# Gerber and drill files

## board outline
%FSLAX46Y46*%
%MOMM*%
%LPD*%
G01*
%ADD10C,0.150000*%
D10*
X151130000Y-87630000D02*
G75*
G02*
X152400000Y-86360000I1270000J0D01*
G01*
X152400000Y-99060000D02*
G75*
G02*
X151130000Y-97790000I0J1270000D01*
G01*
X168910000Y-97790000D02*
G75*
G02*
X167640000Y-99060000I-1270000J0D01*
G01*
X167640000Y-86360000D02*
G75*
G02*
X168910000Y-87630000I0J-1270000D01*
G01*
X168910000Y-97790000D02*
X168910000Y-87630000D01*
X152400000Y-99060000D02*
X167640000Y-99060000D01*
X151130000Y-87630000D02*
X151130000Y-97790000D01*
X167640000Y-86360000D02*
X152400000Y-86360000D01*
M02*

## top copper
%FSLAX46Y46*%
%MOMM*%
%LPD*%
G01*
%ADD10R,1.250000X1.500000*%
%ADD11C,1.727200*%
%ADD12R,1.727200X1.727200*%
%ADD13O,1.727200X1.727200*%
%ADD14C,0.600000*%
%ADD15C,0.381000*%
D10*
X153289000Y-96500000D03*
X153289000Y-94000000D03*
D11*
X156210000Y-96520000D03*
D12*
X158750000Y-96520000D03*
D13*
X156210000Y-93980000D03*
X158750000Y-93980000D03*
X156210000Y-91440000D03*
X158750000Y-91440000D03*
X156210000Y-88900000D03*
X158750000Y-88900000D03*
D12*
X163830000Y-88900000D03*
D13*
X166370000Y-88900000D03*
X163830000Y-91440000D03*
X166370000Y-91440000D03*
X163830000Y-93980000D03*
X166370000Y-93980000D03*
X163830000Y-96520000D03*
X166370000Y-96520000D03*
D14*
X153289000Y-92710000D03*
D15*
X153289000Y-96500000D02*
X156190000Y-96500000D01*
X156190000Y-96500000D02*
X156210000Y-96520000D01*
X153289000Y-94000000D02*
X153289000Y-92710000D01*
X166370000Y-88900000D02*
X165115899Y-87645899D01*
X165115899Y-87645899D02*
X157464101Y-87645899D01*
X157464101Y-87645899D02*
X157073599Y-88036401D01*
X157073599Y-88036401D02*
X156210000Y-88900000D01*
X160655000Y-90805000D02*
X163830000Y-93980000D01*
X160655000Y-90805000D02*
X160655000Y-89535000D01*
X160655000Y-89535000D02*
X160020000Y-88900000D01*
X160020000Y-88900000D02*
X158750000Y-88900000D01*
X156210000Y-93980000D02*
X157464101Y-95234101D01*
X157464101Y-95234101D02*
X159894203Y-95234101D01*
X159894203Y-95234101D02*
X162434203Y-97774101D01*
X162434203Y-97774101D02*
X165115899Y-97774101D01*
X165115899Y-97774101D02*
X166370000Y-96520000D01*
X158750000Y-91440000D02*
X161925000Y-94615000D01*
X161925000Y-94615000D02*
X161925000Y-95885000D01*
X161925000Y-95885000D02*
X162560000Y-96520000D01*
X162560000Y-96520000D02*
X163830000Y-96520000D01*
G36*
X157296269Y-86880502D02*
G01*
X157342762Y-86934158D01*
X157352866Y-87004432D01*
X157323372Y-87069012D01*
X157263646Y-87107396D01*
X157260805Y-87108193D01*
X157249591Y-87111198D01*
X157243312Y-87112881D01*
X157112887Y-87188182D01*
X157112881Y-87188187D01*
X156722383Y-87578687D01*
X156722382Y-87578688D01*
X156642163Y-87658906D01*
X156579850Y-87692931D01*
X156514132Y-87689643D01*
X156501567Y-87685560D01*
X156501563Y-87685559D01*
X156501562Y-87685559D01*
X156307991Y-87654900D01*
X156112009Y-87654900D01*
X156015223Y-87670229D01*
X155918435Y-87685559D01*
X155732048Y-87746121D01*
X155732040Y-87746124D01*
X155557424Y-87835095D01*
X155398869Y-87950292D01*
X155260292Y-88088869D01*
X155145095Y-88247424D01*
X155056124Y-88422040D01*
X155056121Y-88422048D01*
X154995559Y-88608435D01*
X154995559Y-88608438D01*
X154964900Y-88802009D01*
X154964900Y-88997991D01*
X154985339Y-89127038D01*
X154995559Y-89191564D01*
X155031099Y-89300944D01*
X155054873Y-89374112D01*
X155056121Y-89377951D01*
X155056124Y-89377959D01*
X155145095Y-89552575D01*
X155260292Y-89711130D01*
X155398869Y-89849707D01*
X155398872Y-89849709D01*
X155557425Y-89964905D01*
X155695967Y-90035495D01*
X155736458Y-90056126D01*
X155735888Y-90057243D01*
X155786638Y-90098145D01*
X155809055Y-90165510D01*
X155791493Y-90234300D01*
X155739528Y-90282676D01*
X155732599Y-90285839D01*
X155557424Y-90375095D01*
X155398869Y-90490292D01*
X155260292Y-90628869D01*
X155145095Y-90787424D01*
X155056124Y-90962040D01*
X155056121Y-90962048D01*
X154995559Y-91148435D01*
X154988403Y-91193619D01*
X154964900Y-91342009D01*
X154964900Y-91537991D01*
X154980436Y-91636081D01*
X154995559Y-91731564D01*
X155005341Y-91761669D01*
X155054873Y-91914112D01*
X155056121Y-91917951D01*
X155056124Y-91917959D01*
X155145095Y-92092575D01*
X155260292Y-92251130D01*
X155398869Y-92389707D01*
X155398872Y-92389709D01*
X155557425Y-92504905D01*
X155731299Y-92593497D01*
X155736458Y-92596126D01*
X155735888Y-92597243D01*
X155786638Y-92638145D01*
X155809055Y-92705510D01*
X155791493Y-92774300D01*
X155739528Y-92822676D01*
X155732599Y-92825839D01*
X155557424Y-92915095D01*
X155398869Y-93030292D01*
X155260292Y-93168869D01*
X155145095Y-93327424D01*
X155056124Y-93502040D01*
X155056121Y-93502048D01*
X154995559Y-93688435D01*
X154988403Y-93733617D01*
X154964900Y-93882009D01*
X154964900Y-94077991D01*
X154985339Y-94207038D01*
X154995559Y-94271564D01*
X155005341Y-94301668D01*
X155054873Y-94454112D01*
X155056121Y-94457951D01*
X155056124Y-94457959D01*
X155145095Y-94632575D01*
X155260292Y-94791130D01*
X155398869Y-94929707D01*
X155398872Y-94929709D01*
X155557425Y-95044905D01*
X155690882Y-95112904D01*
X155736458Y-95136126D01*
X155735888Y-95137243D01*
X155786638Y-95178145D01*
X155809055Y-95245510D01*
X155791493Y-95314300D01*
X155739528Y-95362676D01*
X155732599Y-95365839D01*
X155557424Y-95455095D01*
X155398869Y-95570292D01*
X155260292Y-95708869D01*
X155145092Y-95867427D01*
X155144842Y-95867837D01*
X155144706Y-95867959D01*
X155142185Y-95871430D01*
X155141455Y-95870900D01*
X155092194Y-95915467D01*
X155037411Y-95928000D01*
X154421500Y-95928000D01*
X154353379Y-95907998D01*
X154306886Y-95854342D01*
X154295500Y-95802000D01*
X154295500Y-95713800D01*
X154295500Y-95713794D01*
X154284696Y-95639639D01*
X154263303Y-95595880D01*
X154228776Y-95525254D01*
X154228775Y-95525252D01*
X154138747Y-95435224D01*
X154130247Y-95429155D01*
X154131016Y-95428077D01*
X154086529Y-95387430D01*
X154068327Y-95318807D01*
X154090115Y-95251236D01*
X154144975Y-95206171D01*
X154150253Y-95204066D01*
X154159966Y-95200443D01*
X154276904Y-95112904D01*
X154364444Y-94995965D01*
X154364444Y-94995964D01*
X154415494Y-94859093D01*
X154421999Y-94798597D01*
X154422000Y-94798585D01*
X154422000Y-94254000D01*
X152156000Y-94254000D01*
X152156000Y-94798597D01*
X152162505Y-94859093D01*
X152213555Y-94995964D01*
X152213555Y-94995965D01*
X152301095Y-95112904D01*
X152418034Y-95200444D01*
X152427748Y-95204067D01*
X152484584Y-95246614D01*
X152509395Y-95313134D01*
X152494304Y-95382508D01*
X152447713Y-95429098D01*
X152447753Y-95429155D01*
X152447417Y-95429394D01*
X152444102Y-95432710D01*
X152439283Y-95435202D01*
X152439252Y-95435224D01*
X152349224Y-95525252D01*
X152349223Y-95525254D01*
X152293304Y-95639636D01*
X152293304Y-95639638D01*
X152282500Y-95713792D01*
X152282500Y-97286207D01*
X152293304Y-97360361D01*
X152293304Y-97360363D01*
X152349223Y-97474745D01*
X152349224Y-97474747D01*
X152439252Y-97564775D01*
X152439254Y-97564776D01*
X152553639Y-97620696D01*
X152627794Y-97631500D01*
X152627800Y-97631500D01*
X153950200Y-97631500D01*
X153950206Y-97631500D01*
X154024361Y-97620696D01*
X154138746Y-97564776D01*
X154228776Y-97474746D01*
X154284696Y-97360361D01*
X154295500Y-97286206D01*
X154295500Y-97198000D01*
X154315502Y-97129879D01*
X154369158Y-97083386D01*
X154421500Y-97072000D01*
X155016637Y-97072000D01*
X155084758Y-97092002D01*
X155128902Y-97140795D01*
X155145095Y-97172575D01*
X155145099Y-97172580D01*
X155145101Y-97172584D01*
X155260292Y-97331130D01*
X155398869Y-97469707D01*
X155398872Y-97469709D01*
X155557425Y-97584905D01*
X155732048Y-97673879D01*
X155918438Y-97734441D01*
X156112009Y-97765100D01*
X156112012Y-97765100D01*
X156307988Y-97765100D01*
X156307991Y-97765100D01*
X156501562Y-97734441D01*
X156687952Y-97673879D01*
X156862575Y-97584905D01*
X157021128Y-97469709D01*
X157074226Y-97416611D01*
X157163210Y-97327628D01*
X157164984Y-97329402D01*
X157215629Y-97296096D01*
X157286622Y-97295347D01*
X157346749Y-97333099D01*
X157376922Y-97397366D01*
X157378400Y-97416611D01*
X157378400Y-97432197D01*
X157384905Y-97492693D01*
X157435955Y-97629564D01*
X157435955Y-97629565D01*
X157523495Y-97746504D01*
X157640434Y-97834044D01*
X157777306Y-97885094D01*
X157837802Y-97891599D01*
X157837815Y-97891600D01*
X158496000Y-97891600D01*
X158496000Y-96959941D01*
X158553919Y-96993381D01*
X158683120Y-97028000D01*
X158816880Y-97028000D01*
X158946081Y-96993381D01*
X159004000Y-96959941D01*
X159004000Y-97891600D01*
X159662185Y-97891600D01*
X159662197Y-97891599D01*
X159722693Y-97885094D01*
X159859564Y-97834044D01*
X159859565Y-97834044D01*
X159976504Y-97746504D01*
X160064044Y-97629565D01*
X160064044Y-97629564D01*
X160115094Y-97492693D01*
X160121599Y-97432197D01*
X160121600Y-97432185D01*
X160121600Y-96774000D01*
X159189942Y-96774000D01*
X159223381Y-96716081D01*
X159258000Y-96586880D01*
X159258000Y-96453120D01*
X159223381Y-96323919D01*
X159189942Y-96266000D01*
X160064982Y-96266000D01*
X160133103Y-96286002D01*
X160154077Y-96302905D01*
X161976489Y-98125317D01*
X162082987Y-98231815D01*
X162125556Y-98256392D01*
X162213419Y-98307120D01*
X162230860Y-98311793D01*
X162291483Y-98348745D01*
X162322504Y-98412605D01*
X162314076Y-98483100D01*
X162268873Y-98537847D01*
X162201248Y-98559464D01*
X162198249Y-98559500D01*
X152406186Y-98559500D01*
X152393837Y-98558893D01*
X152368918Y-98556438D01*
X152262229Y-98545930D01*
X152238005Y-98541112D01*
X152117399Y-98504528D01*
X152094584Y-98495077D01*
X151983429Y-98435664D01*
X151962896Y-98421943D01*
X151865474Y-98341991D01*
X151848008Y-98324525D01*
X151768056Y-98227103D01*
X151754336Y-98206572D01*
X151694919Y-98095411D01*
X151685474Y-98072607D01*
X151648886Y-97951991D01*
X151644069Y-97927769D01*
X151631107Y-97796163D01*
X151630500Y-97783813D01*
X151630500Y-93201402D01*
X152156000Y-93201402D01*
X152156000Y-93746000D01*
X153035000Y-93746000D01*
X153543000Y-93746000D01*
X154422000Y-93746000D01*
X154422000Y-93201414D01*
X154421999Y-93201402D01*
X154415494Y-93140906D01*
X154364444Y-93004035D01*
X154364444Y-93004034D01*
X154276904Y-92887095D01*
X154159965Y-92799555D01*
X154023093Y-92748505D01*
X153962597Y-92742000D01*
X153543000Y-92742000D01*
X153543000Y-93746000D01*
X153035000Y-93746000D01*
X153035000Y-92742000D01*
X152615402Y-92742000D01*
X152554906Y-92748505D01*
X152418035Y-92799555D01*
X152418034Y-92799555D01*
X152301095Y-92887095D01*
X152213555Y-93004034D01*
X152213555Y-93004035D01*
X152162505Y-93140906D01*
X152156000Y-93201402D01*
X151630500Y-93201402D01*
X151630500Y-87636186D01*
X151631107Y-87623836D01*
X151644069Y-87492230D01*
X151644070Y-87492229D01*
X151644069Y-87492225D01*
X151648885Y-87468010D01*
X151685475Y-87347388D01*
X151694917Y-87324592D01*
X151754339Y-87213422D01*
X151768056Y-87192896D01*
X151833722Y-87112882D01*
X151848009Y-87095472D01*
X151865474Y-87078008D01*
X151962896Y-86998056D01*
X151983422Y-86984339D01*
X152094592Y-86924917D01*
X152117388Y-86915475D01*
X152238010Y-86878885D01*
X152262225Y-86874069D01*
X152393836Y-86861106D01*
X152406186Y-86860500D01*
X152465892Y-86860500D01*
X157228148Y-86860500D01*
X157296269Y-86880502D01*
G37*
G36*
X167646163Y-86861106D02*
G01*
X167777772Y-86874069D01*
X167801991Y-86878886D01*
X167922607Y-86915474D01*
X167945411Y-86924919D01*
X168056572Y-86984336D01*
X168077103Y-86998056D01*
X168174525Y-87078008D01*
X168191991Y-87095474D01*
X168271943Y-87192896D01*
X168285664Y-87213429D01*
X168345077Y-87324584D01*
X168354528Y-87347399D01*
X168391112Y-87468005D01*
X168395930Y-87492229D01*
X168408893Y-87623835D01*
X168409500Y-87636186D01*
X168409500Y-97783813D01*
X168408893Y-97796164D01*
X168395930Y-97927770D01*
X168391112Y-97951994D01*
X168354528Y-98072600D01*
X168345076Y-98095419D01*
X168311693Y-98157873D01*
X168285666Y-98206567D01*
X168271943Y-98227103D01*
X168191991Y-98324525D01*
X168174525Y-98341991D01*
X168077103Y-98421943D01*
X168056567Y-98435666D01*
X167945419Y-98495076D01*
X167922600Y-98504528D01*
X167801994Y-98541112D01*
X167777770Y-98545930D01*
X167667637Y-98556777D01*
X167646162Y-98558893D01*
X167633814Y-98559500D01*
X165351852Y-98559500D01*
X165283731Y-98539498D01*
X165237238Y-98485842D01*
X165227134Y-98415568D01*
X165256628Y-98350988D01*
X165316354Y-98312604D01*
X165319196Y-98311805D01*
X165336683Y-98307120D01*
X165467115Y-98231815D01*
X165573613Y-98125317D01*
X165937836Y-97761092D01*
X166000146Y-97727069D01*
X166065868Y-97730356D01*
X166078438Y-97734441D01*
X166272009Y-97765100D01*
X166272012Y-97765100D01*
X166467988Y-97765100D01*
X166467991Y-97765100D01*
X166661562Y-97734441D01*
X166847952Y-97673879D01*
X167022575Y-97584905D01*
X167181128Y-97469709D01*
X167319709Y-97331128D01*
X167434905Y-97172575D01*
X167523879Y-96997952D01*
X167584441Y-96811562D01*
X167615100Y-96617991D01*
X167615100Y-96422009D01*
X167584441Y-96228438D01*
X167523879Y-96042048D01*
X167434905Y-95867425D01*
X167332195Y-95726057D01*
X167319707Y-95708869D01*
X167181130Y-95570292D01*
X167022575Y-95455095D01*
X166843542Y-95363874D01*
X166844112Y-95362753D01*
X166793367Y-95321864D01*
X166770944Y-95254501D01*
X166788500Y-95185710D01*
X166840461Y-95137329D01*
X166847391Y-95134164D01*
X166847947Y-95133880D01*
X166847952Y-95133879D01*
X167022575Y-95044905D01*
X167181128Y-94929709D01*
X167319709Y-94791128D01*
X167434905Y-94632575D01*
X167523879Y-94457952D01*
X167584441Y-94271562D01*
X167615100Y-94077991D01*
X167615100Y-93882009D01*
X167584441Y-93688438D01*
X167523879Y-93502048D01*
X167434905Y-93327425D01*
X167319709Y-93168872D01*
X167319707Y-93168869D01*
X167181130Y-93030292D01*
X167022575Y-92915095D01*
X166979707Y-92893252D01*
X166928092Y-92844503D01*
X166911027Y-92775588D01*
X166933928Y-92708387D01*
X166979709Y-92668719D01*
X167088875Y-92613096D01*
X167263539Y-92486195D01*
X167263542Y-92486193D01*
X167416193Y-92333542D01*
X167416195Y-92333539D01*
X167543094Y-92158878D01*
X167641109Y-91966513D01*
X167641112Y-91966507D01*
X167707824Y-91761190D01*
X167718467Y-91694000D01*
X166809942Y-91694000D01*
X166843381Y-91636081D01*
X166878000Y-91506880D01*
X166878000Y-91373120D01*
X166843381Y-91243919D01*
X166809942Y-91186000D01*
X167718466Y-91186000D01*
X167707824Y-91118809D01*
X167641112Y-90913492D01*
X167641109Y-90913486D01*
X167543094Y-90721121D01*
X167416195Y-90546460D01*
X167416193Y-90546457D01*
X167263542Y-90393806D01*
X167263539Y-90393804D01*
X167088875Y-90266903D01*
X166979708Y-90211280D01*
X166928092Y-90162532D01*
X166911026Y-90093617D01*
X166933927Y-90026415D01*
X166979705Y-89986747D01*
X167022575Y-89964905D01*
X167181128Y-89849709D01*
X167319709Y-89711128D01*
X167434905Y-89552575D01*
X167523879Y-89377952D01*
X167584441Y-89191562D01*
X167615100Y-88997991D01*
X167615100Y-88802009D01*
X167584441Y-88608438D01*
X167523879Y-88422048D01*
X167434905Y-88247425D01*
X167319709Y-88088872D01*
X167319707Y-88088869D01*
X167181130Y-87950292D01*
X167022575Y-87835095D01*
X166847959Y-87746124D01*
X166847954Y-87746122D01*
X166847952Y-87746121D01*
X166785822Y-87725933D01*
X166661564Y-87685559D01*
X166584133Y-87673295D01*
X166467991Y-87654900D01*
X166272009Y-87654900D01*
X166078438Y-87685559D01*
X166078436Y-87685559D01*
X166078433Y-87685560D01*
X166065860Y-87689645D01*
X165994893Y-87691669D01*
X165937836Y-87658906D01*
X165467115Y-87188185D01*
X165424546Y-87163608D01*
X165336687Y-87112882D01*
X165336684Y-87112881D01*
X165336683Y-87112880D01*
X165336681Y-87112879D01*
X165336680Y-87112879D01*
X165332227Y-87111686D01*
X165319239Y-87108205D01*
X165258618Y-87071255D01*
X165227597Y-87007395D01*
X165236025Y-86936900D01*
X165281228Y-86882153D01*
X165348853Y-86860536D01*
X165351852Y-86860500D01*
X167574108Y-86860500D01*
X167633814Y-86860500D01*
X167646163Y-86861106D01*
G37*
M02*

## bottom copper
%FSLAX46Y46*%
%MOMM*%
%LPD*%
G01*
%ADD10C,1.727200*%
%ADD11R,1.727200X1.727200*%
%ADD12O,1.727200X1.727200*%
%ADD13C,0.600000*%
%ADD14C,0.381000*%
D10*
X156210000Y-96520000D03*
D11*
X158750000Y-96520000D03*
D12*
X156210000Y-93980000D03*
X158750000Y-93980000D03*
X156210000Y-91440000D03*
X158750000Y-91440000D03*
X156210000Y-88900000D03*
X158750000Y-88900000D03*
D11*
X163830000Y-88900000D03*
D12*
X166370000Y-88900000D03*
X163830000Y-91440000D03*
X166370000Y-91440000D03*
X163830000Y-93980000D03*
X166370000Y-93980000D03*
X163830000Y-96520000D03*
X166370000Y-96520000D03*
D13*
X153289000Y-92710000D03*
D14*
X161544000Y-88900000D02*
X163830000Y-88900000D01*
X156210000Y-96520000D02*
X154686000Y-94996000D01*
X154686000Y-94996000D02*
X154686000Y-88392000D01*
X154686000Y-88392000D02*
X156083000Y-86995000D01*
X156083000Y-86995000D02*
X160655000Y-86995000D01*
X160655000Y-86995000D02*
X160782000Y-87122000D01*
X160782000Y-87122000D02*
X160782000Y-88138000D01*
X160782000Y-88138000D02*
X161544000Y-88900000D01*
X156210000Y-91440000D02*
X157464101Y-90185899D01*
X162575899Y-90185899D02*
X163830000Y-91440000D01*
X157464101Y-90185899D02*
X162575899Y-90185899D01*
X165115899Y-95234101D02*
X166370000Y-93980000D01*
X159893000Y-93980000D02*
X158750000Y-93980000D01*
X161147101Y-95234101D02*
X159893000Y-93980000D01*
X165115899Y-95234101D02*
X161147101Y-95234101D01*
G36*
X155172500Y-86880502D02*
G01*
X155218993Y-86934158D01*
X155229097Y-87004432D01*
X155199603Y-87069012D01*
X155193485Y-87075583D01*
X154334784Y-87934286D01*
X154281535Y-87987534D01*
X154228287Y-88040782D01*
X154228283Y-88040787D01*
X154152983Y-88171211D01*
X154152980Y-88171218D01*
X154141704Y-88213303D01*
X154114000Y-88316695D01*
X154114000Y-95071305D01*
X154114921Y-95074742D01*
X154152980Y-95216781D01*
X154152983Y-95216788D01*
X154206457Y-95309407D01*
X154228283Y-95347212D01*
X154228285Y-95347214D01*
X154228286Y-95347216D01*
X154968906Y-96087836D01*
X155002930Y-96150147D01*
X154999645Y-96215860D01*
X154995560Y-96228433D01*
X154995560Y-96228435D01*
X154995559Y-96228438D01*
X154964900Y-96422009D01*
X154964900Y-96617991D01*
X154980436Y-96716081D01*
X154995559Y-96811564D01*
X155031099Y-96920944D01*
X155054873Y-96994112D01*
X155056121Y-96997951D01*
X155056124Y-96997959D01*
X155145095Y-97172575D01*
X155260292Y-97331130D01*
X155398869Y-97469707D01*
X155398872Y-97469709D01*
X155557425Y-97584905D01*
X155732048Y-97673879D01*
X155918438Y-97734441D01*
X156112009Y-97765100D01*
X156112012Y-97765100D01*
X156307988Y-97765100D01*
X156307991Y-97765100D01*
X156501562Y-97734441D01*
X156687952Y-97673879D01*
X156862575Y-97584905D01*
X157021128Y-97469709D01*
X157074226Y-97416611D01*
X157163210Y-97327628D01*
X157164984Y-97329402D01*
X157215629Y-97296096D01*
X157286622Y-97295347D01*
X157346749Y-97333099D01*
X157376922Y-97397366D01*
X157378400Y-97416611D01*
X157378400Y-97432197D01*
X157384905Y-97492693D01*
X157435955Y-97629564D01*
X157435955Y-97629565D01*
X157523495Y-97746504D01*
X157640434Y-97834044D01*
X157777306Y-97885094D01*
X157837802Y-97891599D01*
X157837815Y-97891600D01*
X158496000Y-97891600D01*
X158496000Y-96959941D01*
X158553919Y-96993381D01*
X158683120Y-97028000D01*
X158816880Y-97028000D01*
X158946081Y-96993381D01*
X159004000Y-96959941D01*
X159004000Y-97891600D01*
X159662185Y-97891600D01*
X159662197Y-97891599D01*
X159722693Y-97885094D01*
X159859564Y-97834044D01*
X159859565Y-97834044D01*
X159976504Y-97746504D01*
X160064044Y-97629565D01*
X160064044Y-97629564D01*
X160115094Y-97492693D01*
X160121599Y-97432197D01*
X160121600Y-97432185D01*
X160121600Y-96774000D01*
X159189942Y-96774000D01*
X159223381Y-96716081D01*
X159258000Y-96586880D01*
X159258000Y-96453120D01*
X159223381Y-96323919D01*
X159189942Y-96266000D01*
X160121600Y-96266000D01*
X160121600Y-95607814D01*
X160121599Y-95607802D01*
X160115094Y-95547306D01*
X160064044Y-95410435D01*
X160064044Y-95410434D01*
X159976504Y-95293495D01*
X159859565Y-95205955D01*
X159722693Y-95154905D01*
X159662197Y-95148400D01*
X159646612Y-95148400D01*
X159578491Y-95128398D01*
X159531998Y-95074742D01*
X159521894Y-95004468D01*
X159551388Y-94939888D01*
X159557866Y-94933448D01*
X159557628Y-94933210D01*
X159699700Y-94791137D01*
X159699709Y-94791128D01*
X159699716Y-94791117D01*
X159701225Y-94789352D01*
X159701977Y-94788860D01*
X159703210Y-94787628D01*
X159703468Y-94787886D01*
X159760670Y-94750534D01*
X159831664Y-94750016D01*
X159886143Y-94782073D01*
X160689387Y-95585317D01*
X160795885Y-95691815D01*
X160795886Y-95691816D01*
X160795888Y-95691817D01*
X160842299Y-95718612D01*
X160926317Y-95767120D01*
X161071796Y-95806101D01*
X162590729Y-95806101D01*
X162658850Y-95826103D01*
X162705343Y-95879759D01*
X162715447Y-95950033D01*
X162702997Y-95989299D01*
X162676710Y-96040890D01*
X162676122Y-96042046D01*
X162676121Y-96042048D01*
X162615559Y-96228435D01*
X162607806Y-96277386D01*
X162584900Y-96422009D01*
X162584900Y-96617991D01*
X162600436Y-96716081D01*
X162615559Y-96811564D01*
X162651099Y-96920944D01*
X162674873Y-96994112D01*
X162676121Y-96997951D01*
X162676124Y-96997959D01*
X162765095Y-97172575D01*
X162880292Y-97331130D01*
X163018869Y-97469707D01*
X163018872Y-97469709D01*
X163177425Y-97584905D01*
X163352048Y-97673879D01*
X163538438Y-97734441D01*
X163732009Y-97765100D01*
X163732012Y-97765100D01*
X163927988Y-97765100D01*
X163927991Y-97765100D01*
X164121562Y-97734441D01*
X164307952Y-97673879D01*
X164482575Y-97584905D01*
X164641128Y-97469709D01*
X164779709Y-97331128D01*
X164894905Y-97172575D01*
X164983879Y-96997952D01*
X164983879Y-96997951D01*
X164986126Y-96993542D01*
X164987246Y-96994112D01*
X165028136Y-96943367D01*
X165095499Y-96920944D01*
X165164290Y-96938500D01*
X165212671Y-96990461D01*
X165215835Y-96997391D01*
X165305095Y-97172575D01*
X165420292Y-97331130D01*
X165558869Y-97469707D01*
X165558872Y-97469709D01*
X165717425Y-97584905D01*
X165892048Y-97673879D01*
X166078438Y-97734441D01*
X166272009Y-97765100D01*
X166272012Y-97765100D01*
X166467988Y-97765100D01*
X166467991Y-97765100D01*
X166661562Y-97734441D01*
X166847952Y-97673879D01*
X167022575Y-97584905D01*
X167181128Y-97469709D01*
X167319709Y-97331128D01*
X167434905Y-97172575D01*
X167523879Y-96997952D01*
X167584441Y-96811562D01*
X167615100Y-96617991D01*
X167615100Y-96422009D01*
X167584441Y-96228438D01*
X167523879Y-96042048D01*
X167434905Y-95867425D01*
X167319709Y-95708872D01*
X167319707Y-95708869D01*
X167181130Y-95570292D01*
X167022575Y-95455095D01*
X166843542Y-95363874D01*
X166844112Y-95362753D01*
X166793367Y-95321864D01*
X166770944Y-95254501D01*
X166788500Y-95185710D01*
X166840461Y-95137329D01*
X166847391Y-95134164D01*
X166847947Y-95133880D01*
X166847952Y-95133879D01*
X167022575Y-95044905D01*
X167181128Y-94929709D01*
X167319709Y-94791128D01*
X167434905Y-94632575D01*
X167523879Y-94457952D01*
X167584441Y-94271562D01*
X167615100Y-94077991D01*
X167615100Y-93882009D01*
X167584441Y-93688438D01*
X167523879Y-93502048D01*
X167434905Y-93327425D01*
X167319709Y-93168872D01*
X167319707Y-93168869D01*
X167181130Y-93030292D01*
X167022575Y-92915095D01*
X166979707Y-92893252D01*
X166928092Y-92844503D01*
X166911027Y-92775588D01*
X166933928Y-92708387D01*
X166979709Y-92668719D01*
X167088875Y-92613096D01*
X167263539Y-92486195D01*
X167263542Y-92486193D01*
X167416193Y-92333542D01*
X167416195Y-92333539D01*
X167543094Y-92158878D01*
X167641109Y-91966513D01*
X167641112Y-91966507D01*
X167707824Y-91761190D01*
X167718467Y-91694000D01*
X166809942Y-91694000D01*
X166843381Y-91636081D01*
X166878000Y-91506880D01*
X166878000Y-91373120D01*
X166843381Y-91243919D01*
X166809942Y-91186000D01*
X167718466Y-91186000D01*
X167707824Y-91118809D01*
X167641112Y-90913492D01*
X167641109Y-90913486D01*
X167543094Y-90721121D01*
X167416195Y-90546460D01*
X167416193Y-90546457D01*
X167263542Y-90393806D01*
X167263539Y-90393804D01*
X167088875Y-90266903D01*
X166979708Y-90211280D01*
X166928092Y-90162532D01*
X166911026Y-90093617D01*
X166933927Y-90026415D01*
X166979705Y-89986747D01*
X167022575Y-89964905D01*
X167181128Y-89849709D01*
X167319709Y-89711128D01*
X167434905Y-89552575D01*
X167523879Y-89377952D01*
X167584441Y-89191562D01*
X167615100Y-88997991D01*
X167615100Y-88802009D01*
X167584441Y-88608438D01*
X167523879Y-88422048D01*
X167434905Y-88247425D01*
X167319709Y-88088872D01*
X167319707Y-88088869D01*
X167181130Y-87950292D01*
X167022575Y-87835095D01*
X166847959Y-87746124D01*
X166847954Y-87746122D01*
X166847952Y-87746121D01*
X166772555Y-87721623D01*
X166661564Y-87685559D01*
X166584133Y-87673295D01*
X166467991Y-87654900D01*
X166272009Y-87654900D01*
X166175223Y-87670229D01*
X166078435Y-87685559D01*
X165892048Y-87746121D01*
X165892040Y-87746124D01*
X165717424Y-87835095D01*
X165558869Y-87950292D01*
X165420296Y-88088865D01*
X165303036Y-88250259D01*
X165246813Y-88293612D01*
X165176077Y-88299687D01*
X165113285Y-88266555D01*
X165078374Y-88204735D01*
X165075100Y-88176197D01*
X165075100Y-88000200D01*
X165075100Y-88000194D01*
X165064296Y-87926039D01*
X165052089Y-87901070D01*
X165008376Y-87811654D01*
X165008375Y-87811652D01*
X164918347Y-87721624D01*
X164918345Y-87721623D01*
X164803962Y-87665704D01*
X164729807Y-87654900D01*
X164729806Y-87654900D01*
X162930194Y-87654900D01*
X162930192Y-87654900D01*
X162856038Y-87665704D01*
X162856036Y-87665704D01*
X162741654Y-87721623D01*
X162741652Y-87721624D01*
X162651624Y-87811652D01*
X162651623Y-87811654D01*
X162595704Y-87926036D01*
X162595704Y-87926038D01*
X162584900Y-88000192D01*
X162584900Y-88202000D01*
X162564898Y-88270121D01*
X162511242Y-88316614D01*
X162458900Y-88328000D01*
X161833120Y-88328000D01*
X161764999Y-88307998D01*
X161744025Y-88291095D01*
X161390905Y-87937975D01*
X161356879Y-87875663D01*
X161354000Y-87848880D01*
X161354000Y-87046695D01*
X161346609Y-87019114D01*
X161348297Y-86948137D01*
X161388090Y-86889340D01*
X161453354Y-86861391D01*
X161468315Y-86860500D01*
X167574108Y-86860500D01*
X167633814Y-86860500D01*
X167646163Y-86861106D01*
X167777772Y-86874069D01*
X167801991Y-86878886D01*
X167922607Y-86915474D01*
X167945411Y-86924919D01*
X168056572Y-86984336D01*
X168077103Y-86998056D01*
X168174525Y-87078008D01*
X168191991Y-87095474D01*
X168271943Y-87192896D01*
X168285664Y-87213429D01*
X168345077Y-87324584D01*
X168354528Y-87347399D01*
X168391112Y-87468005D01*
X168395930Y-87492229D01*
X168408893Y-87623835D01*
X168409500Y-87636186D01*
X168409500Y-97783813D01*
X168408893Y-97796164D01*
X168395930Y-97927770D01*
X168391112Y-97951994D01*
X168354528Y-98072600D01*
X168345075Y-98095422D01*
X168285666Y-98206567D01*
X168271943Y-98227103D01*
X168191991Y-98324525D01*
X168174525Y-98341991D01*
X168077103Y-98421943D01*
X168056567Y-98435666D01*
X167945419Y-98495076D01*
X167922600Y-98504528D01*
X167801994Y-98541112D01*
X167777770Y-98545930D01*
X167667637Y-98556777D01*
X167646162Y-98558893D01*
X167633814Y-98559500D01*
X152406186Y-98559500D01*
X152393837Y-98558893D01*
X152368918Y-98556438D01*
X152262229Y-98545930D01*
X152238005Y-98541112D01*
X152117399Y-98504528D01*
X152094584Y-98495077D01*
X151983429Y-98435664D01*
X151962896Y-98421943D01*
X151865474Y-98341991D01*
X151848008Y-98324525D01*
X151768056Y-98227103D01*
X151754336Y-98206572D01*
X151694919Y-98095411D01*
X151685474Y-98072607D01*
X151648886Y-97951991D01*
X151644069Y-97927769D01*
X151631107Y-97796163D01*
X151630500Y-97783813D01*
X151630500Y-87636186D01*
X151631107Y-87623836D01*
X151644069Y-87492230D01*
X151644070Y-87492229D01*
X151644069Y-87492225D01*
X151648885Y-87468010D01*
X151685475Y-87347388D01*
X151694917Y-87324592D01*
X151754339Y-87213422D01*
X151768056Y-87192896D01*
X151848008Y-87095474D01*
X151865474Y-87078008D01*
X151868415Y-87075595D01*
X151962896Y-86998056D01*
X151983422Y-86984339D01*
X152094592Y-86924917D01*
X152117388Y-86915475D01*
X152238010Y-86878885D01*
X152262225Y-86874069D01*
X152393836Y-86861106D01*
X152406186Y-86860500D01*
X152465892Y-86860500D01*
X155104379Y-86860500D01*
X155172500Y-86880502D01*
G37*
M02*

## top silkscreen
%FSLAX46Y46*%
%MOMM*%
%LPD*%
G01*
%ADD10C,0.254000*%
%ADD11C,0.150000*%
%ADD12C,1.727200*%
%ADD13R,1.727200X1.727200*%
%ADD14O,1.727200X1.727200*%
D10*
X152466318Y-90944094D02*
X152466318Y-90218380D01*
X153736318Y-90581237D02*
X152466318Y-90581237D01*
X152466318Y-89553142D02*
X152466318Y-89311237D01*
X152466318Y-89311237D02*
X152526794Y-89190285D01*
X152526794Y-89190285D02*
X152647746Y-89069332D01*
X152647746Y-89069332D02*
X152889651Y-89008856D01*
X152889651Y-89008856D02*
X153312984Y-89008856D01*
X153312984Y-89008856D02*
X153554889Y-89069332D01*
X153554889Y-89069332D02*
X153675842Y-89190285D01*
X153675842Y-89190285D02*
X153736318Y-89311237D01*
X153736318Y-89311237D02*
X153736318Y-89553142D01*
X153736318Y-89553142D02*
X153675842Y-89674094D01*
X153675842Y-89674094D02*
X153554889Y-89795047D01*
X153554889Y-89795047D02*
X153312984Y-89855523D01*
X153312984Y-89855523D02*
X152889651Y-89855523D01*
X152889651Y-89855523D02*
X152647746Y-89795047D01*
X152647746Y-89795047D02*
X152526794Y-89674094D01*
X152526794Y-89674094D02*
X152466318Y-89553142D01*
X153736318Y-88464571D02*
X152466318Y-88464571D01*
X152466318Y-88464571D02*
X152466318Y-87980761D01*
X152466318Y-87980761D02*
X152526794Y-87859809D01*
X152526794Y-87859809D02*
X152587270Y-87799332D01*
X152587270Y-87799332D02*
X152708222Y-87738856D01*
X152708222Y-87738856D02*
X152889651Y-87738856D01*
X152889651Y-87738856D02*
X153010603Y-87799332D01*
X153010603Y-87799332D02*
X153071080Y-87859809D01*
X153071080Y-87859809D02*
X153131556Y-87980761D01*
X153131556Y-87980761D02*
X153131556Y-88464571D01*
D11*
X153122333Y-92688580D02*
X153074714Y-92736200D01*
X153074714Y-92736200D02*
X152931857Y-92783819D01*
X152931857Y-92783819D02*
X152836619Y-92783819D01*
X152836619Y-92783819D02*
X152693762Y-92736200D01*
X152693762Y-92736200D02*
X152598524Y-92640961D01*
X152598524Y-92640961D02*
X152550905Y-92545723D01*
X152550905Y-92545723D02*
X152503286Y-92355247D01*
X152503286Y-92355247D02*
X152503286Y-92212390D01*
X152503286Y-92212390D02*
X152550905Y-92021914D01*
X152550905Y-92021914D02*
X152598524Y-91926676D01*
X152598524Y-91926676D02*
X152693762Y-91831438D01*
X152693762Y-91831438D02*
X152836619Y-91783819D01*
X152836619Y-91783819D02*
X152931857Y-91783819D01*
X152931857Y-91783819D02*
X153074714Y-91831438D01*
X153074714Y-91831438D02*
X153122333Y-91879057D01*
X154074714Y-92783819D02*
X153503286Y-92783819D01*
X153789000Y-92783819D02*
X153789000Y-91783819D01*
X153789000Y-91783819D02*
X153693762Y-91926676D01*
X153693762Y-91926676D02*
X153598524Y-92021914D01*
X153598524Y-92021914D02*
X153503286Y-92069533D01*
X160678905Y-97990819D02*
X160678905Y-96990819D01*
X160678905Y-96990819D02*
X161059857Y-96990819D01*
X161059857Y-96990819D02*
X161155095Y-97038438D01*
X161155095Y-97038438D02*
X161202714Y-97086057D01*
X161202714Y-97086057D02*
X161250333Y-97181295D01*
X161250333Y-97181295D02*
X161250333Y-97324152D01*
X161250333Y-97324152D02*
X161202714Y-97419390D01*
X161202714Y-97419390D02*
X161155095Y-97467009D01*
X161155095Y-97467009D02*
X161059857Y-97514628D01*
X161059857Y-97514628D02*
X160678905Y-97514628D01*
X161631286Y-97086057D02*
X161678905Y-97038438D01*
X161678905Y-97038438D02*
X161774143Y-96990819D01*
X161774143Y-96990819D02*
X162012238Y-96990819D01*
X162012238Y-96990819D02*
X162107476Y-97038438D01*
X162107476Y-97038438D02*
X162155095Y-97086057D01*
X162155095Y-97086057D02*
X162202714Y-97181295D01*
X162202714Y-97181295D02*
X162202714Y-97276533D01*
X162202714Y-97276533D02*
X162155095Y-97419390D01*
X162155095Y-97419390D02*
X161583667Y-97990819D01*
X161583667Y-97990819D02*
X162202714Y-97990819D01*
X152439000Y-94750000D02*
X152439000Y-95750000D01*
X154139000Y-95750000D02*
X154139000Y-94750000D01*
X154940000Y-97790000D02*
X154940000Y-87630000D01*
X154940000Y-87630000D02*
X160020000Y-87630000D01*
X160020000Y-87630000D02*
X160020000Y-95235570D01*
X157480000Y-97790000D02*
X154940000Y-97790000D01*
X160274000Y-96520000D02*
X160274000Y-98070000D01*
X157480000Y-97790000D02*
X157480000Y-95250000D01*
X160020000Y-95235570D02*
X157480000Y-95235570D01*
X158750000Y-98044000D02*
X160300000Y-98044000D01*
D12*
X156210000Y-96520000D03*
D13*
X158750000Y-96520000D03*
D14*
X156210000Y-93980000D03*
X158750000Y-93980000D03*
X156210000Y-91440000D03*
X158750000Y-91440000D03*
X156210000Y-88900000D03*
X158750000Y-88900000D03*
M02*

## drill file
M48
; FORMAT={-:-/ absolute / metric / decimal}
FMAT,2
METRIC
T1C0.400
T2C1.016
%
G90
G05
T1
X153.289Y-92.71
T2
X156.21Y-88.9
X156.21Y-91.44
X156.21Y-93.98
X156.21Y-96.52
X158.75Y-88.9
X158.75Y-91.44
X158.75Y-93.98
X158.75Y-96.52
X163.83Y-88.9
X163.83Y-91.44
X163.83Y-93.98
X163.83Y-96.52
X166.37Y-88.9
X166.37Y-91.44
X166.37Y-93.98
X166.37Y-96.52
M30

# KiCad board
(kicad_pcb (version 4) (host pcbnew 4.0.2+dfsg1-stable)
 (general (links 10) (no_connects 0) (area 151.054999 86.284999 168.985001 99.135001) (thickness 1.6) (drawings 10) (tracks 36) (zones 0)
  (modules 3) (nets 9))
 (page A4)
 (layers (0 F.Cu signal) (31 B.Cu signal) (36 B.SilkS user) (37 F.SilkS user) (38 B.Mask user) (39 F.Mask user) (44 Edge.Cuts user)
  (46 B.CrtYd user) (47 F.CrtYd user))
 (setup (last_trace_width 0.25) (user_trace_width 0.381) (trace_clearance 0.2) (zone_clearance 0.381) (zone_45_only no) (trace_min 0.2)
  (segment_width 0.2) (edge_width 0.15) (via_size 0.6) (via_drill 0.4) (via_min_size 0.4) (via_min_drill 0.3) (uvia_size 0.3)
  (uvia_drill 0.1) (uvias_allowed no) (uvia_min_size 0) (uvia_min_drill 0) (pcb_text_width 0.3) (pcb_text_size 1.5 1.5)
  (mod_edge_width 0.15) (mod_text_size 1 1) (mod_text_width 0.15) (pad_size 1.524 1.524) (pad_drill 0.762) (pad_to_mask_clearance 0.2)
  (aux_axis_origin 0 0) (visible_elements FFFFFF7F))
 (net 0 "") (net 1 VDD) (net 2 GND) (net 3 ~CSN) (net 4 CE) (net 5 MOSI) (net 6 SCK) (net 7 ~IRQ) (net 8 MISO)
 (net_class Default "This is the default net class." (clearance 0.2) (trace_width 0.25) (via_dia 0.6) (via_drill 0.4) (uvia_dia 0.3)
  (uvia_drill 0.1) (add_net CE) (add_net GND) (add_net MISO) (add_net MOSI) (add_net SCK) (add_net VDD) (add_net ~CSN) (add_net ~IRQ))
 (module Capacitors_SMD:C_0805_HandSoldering (layer F.Cu) (at 153.289 95.25 90)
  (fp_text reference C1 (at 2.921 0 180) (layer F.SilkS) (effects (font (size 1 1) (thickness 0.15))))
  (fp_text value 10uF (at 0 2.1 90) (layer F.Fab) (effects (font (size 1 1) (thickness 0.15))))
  (fp_line (start 0.5 -0.85) (end -0.5 -0.85) (layer F.SilkS) (width 0.15))
  (fp_line (start -0.5 0.85) (end 0.5 0.85) (layer F.SilkS) (width 0.15))
  (pad 1 smd rect (at -1.25 0 90) (size 1.5 1.25) (layers F.Cu F.Mask) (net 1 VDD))
  (pad 2 smd rect (at 1.25 0 90) (size 1.5 1.25) (layers F.Cu F.Mask) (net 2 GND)))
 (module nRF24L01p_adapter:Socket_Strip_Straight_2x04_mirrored (layer F.Cu) (at 156.21 96.52 90)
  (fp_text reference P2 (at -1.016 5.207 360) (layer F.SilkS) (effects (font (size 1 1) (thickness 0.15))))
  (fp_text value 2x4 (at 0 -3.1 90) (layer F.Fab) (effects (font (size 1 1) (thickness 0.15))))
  (fp_line (start -1.27 -1.27) (end 8.89 -1.27) (layer F.SilkS) (width 0.15))
  (fp_line (start 8.89 -1.27) (end 8.89 3.81) (layer F.SilkS) (width 0.15))
  (fp_line (start 8.89 3.81) (end 1.28443 3.81) (layer F.SilkS) (width 0.15))
  (fp_line (start -1.27 1.27) (end -1.27 -1.27) (layer F.SilkS) (width 0.15))
  (fp_line (start 0 4.064) (end -1.55 4.064) (layer F.SilkS) (width 0.15))
  (fp_line (start -1.27 1.27) (end 1.27 1.27) (layer F.SilkS) (width 0.15))
  (fp_line (start 1.28443 3.81) (end 1.28443 1.27) (layer F.SilkS) (width 0.15))
  (fp_line (start -1.524 2.54) (end -1.524 4.09) (layer F.SilkS) (width 0.15))
  (pad 2 thru_hole circle (at 0 0 90) (size 1.7272 1.7272) (drill 1.016) (layers *.Cu *.Mask F.SilkS) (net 1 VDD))
  (pad 1 thru_hole rect (at 0 2.54 90) (size 1.7272 1.7272) (drill 1.016) (layers *.Cu *.Mask F.SilkS) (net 2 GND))
  (pad 4 thru_hole oval (at 2.54 0 90) (size 1.7272 1.7272) (drill 1.016) (layers *.Cu *.Mask F.SilkS) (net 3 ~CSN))
  (pad 3 thru_hole oval (at 2.54 2.54 90) (size 1.7272 1.7272) (drill 1.016) (layers *.Cu *.Mask F.SilkS) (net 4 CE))
  (pad 6 thru_hole oval (at 5.08 0 90) (size 1.7272 1.7272) (drill 1.016) (layers *.Cu *.Mask F.SilkS) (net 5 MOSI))
  (pad 5 thru_hole oval (at 5.08 2.54 90) (size 1.7272 1.7272) (drill 1.016) (layers *.Cu *.Mask F.SilkS) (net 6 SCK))
  (pad 8 thru_hole oval (at 7.62 0 90) (size 1.7272 1.7272) (drill 1.016) (layers *.Cu *.Mask F.SilkS) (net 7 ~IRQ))
  (pad 7 thru_hole oval (at 7.62 2.54 90) (size 1.7272 1.7272) (drill 1.016) (layers *.Cu *.Mask F.SilkS) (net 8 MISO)))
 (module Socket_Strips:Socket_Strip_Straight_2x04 (layer B.Cu) (at 163.83 88.9 270)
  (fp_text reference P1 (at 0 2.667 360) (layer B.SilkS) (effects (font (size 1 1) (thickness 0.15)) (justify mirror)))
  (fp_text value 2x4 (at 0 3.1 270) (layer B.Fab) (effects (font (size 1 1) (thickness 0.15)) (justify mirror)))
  (pad 1 thru_hole rect (at 0 0 270) (size 1.7272 1.7272) (drill 1.016) (layers *.Cu *.Mask B.SilkS) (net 1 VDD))
  (pad 2 thru_hole oval (at 0 -2.54 270) (size 1.7272 1.7272) (drill 1.016) (layers *.Cu *.Mask B.SilkS) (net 7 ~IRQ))
  (pad 3 thru_hole oval (at 2.54 0 270) (size 1.7272 1.7272) (drill 1.016) (layers *.Cu *.Mask B.SilkS) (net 5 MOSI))
  (pad 4 thru_hole oval (at 2.54 -2.54 270) (size 1.7272 1.7272) (drill 1.016) (layers *.Cu *.Mask B.SilkS) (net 2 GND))
  (pad 5 thru_hole oval (at 5.08 0 270) (size 1.7272 1.7272) (drill 1.016) (layers *.Cu *.Mask B.SilkS) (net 8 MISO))
  (pad 6 thru_hole oval (at 5.08 -2.54 270) (size 1.7272 1.7272) (drill 1.016) (layers *.Cu *.Mask B.SilkS) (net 4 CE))
  (pad 7 thru_hole oval (at 7.62 0 270) (size 1.7272 1.7272) (drill 1.016) (layers *.Cu *.Mask B.SilkS) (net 6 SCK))
  (pad 8 thru_hole oval (at 7.62 -2.54 270) (size 1.7272 1.7272) (drill 1.016) (layers *.Cu *.Mask B.SilkS) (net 3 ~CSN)))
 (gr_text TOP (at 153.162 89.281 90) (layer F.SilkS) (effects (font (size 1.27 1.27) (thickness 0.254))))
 (gr_arc (start 152.4 87.63) (end 151.13 87.63) (angle 90) (layer Edge.Cuts) (width 0.15))
 (gr_arc (start 152.4 97.79) (end 152.4 99.06) (angle 90) (layer Edge.Cuts) (width 0.15))
 (gr_arc (start 167.64 97.79) (end 168.91 97.79) (angle 90) (layer Edge.Cuts) (width 0.15))
 (gr_arc (start 167.64 87.63) (end 167.64 86.36) (angle 90) (layer Edge.Cuts) (width 0.15))
 (gr_line (start 168.91 97.79) (end 168.91 87.63) (layer Edge.Cuts) (width 0.15))
 (gr_line (start 152.4 99.06) (end 167.64 99.06) (layer Edge.Cuts) (width 0.15))
 (gr_line (start 151.13 87.63) (end 151.13 97.79) (layer Edge.Cuts) (width 0.15))
 (gr_line (start 167.64 86.36) (end 152.4 86.36) (layer Edge.Cuts) (width 0.15))
 (segment (start 153.289 96.5) (end 156.19 96.5) (width 0.381) (layer F.Cu) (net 1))
 (segment (start 156.19 96.5) (end 156.21 96.52) (width 0.381) (layer F.Cu) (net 1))
 (segment (start 161.544 88.9) (end 163.83 88.9) (width 0.381) (layer B.Cu) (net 1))
 (segment (start 156.21 96.52) (end 154.686 94.996) (width 0.381) (layer B.Cu) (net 1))
 (segment (start 154.686 94.996) (end 154.686 88.392) (width 0.381) (layer B.Cu) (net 1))
 (segment (start 154.686 88.392) (end 156.083 86.995) (width 0.381) (layer B.Cu) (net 1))
 (segment (start 156.083 86.995) (end 160.655 86.995) (width 0.381) (layer B.Cu) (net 1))
 (segment (start 160.655 86.995) (end 160.782 87.122) (width 0.381) (layer B.Cu) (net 1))
 (segment (start 160.782 87.122) (end 160.782 88.138) (width 0.381) (layer B.Cu) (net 1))
 (segment (start 160.782 88.138) (end 161.544 88.9) (width 0.381) (layer B.Cu) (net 1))
 (segment (start 153.289 94) (end 153.289 92.71) (width 0.381) (layer F.Cu) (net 2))
 (via (at 153.289 92.71) (size 0.6) (drill 0.4) (layers F.Cu B.Cu) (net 2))
 (segment (start 166.37 88.9) (end 165.115899 87.645899) (width 0.381) (layer F.Cu) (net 7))
 (segment (start 165.115899 87.645899) (end 157.464101 87.645899) (width 0.381) (layer F.Cu) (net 7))
 (segment (start 157.464101 87.645899) (end 157.073599 88.036401) (width 0.381) (layer F.Cu) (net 7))
 (segment (start 157.073599 88.036401) (end 156.21 88.9) (width 0.381) (layer F.Cu) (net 7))
 (segment (start 156.21 91.44) (end 157.464101 90.185899) (width 0.381) (layer B.Cu) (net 5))
 (segment (start 162.575899 90.185899) (end 163.83 91.44) (width 0.381) (layer B.Cu) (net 5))
 (segment (start 157.464101 90.185899) (end 162.575899 90.185899) (width 0.381) (layer B.Cu) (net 5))
 (segment (start 165.115899 95.234101) (end 166.37 93.98) (width 0.381) (layer B.Cu) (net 4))
 (segment (start 159.893 93.98) (end 158.75 93.98) (width 0.381) (layer B.Cu) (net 4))
 (segment (start 161.147101 95.234101) (end 159.893 93.98) (width 0.381) (layer B.Cu) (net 4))
 (segment (start 165.115899 95.234101) (end 161.147101 95.234101) (width 0.381) (layer B.Cu) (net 4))
 (segment (start 160.655 90.805) (end 163.83 93.98) (width 0.381) (layer F.Cu) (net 8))
 (segment (start 160.655 90.805) (end 160.655 89.535) (width 0.381) (layer F.Cu) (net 8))
 (segment (start 160.655 89.535) (end 160.02 88.9) (width 0.381) (layer F.Cu) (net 8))
 (segment (start 160.02 88.9) (end 158.75 88.9) (width 0.381) (layer F.Cu) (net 8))
 (segment (start 156.21 93.98) (end 157.464101 95.234101) (width 0.381) (layer F.Cu) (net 3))
 (segment (start 157.464101 95.234101) (end 159.894203 95.234101) (width 0.381) (layer F.Cu) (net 3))
 (segment (start 159.894203 95.234101) (end 162.434203 97.774101) (width 0.381) (layer F.Cu) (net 3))
 (segment (start 162.434203 97.774101) (end 165.115899 97.774101) (width 0.381) (layer F.Cu) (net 3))
 (segment (start 165.115899 97.774101) (end 166.37 96.52) (width 0.381) (layer F.Cu) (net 3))
 (segment (start 158.75 91.44) (end 161.925 94.615) (width 0.381) (layer F.Cu) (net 6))
 (segment (start 161.925 94.615) (end 161.925 95.885) (width 0.381) (layer F.Cu) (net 6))
 (segment (start 161.925 95.885) (end 162.56 96.52) (width 0.381) (layer F.Cu) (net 6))
 (segment (start 162.56 96.52) (end 163.83 96.52) (width 0.381) (layer F.Cu) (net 6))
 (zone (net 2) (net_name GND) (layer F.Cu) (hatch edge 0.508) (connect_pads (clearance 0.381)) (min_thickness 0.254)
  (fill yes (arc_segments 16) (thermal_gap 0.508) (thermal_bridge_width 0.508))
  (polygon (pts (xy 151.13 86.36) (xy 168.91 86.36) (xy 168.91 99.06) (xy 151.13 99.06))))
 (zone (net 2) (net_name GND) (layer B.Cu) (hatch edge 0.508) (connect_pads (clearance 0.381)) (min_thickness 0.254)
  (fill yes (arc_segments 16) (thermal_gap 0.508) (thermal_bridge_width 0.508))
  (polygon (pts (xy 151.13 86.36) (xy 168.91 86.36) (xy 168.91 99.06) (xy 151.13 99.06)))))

